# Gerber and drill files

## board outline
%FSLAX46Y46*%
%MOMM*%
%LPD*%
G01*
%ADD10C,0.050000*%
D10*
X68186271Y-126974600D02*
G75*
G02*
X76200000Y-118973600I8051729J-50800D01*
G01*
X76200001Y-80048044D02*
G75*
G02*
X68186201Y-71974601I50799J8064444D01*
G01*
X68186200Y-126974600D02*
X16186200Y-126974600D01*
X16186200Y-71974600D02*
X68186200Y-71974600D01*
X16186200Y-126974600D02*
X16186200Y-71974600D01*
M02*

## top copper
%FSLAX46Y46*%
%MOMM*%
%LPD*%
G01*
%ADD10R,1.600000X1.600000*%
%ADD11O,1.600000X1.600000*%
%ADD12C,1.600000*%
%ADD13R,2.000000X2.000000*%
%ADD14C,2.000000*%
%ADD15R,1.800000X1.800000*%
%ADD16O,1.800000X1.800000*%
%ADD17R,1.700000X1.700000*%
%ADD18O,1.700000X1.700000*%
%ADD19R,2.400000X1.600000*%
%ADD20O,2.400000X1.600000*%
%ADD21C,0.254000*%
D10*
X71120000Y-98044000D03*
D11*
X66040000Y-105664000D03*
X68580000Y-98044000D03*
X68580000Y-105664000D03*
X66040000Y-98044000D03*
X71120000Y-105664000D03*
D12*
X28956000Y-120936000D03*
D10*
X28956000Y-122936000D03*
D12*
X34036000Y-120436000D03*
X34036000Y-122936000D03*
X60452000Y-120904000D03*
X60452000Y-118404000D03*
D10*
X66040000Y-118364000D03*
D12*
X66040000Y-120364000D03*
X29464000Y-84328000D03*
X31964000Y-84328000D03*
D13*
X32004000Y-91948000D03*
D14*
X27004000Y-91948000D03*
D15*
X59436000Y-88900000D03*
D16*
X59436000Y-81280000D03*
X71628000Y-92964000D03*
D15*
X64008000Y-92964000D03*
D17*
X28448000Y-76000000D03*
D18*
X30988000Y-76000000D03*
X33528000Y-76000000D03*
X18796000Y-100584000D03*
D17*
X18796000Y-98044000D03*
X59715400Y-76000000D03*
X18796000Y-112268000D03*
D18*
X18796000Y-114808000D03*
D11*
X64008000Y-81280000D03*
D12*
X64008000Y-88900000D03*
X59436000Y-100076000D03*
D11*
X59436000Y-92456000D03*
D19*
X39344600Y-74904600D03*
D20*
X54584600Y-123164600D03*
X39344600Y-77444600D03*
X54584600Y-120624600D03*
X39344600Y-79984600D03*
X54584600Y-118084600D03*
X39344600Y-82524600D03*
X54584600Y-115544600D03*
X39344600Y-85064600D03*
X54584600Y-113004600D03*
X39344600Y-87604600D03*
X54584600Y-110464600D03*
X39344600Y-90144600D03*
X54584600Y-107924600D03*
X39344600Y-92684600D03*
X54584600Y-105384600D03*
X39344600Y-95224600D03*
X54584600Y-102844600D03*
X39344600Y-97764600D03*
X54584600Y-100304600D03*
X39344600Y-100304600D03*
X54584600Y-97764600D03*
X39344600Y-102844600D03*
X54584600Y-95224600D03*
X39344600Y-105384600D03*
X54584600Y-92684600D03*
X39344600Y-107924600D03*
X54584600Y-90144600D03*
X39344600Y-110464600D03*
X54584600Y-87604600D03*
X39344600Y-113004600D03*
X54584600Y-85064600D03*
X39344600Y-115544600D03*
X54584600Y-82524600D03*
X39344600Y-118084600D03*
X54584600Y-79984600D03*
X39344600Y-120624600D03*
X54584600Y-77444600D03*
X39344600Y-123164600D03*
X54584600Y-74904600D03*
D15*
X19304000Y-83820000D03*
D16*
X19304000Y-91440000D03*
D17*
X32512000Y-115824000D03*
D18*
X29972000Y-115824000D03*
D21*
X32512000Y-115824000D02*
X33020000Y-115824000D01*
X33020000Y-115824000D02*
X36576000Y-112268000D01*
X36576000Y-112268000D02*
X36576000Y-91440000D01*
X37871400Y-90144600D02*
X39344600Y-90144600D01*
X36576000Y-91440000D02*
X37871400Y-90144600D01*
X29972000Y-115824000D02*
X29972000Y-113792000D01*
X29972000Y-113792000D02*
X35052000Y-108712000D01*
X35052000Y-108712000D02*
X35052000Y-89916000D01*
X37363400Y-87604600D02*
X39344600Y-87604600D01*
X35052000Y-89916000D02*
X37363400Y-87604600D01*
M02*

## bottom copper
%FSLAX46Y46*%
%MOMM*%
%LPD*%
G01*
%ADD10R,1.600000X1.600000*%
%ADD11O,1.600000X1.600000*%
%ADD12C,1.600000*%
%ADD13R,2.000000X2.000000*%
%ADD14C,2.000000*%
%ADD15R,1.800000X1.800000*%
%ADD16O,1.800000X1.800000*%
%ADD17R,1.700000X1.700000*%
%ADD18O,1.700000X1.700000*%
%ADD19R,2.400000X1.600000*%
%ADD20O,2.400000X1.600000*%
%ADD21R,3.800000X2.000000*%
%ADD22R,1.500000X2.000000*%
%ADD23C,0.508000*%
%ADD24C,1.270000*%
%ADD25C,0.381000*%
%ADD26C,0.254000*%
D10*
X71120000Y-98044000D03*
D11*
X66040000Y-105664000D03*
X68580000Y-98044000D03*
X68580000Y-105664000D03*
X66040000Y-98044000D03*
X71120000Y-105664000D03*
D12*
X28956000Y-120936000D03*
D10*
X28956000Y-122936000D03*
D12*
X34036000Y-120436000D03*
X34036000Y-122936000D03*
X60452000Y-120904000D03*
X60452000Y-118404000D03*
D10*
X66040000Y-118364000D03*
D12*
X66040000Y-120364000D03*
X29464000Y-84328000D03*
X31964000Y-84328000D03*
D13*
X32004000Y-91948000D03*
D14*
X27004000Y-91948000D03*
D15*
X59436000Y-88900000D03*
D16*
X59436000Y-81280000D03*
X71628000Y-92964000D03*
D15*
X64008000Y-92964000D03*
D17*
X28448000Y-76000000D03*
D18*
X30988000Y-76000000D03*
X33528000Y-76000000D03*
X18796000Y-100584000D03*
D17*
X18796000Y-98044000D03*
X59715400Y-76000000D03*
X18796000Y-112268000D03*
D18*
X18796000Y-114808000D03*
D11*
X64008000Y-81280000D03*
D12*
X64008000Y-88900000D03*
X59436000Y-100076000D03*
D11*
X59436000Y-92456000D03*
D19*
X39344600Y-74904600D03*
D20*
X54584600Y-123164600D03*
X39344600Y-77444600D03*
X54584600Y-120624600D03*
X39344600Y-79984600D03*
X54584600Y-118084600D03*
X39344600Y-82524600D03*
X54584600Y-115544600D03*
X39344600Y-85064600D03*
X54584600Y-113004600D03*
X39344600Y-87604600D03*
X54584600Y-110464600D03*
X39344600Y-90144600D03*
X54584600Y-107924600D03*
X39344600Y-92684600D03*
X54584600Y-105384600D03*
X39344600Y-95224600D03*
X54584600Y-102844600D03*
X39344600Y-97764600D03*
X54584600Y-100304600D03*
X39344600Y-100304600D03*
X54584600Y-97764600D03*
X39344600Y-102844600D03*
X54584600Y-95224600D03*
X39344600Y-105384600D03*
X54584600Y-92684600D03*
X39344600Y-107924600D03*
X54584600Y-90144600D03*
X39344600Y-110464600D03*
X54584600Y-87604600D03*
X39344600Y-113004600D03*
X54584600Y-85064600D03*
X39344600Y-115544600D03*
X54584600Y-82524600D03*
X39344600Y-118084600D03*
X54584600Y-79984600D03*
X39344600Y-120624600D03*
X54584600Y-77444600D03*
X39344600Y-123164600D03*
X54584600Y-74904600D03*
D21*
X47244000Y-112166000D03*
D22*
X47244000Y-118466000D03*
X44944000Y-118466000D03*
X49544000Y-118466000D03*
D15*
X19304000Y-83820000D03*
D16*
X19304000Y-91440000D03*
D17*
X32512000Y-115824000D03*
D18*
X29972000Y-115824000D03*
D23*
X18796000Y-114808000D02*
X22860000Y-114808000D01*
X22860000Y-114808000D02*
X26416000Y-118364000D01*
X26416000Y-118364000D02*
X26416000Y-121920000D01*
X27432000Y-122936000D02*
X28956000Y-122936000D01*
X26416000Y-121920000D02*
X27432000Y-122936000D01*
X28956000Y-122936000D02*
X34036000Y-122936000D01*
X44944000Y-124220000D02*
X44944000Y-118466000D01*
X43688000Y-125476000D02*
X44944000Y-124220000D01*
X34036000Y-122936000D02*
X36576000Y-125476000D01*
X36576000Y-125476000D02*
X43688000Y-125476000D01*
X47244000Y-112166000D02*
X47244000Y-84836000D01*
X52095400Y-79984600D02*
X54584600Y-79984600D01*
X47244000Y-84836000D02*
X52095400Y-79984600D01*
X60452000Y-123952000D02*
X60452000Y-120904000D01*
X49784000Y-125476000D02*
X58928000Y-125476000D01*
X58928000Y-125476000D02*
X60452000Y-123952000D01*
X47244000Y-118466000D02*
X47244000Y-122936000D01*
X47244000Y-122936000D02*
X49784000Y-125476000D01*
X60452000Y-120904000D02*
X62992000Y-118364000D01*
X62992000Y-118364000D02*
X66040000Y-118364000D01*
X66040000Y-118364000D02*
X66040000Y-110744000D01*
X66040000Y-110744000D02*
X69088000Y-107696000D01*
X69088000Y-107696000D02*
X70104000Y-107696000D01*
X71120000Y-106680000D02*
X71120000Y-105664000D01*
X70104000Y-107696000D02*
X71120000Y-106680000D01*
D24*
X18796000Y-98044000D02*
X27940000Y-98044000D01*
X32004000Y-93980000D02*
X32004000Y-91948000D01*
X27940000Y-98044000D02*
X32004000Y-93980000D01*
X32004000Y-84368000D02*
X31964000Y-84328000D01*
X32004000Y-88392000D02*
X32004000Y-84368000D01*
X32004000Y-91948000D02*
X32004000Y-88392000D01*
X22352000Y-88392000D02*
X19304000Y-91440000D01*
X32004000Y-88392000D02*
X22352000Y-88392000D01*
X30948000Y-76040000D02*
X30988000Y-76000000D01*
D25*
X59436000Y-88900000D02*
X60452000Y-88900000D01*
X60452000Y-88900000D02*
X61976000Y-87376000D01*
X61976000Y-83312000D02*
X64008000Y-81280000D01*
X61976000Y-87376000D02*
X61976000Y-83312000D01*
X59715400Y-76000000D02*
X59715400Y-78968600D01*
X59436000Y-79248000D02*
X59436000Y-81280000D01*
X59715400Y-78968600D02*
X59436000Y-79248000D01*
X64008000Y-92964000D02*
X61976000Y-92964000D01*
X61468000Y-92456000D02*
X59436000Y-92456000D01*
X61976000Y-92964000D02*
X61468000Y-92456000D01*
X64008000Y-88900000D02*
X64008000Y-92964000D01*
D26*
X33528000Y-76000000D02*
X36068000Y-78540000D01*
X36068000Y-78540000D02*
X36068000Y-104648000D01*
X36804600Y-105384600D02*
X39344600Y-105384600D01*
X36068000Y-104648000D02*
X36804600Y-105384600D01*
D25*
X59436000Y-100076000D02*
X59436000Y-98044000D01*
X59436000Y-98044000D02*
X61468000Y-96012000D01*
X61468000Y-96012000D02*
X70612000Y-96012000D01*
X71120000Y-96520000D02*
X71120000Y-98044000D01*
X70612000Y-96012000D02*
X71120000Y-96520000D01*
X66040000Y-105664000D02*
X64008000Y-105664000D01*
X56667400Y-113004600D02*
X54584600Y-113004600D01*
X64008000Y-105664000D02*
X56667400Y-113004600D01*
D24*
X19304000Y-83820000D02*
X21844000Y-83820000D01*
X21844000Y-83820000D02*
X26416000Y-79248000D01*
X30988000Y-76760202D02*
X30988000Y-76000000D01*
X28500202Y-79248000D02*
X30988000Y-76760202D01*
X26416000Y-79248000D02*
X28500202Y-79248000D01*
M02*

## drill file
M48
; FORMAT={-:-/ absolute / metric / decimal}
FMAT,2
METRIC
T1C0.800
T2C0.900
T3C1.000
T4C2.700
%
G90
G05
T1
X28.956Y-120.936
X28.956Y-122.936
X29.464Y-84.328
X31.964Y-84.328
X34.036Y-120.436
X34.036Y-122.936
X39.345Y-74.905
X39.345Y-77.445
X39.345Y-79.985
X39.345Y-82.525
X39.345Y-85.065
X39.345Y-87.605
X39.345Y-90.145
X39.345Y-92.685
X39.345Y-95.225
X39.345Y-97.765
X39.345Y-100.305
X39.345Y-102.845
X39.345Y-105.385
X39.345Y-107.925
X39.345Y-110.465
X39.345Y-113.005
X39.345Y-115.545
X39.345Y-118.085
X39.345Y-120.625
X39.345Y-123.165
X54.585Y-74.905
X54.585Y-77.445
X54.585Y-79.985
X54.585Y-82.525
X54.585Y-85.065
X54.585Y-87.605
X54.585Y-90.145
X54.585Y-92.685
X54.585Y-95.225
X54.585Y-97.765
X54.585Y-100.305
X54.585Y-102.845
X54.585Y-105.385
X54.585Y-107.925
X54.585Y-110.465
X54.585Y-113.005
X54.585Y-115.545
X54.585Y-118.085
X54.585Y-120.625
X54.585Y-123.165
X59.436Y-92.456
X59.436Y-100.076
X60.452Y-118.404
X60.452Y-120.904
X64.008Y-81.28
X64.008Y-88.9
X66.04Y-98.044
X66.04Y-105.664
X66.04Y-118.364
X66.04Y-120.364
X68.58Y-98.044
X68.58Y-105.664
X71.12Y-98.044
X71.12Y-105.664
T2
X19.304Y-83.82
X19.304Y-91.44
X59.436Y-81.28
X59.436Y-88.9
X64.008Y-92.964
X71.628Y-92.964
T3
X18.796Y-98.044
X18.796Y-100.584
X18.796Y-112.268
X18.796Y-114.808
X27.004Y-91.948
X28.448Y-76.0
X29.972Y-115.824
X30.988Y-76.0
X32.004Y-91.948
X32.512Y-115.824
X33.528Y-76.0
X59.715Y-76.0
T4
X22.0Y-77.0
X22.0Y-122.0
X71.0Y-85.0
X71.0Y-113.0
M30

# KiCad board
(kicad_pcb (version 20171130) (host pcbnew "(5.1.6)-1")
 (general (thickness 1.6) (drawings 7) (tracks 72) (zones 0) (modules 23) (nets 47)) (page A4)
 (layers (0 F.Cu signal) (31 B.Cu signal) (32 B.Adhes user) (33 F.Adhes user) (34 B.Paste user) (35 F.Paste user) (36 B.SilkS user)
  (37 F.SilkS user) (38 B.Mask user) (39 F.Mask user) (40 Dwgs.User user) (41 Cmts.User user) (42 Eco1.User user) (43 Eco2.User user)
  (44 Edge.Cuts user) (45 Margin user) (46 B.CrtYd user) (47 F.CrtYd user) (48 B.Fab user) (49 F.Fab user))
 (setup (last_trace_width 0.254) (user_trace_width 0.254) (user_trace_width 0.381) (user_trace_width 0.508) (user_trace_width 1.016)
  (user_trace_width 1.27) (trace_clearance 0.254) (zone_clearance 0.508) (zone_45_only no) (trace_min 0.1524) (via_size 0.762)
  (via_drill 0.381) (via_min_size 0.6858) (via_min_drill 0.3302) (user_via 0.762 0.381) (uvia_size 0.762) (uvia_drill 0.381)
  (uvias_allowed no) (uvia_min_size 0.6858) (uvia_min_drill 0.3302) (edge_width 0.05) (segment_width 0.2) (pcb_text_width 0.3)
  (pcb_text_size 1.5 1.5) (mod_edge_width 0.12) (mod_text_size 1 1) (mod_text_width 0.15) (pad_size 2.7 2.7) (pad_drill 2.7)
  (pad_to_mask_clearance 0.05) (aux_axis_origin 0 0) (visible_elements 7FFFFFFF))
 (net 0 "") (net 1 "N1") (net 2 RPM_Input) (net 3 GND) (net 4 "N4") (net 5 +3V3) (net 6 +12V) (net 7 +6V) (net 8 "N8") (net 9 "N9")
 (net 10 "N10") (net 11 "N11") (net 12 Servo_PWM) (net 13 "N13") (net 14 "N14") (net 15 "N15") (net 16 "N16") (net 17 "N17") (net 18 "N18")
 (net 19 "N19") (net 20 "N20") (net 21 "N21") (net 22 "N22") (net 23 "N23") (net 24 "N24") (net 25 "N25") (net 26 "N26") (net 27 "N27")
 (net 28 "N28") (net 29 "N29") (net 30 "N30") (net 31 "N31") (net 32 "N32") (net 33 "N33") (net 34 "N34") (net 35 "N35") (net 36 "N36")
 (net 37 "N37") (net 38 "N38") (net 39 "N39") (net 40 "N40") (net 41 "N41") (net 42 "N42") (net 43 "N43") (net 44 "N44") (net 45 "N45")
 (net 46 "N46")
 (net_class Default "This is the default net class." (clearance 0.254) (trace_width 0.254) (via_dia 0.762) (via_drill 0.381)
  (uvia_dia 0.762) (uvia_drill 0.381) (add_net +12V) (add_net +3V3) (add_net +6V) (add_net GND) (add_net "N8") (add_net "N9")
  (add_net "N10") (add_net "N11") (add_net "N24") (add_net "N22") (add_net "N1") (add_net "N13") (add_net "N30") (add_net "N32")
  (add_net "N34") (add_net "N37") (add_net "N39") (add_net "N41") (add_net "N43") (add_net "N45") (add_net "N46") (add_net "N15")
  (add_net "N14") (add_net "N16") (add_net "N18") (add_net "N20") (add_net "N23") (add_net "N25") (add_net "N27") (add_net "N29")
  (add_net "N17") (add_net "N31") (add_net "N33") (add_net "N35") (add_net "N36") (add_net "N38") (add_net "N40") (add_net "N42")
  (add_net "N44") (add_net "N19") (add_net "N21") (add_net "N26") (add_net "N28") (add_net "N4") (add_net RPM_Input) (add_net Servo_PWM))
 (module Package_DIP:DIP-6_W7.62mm (layer F.Cu) (at 71.12 98.044 270)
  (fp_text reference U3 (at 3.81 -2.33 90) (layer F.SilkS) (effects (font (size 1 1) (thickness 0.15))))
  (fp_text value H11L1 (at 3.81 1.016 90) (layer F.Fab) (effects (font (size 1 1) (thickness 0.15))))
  (pad 1 thru_hole rect (at 0 0 270) (size 1.6 1.6) (drill 0.8) (layers *.Cu *.Mask) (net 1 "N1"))
  (pad 4 thru_hole oval (at 7.62 5.08 270) (size 1.6 1.6) (drill 0.8) (layers *.Cu *.Mask) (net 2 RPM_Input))
  (pad 2 thru_hole oval (at 0 2.54 270) (size 1.6 1.6) (drill 0.8) (layers *.Cu *.Mask) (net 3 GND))
  (pad 5 thru_hole oval (at 7.62 2.54 270) (size 1.6 1.6) (drill 0.8) (layers *.Cu *.Mask) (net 3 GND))
  (pad 3 thru_hole oval (at 0 5.08 270) (size 1.6 1.6) (drill 0.8) (layers *.Cu *.Mask) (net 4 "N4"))
  (pad 6 thru_hole oval (at 7.62 0 270) (size 1.6 1.6) (drill 0.8) (layers *.Cu *.Mask) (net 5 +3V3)))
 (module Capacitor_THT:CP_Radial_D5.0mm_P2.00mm (layer F.Cu) (at 28.956 122.936 90)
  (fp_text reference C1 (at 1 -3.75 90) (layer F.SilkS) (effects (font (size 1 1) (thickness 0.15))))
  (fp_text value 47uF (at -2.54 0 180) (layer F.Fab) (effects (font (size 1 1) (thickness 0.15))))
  (pad 2 thru_hole circle (at 2 0 90) (size 1.6 1.6) (drill 0.8) (layers *.Cu *.Mask) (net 3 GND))
  (pad 1 thru_hole rect (at 0 0 90) (size 1.6 1.6) (drill 0.8) (layers *.Cu *.Mask) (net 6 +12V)))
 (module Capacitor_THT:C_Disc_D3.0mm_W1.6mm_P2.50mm (layer F.Cu) (at 34.036 122.936 90)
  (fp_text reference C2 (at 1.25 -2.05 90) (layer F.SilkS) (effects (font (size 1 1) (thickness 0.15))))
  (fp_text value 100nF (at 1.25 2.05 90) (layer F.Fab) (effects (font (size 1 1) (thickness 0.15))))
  (pad 2 thru_hole circle (at 2.5 0 90) (size 1.6 1.6) (drill 0.8) (layers *.Cu *.Mask) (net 3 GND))
  (pad 1 thru_hole circle (at 0 0 90) (size 1.6 1.6) (drill 0.8) (layers *.Cu *.Mask) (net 6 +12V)))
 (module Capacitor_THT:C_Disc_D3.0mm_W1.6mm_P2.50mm (layer F.Cu) (at 60.452 120.904 90)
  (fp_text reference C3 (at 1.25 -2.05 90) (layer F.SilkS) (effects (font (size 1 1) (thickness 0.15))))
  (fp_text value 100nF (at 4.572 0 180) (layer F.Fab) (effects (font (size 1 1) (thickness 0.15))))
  (pad 1 thru_hole circle (at 0 0 90) (size 1.6 1.6) (drill 0.8) (layers *.Cu *.Mask) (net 5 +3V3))
  (pad 2 thru_hole circle (at 2.5 0 90) (size 1.6 1.6) (drill 0.8) (layers *.Cu *.Mask) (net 3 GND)))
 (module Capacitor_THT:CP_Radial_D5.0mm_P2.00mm (layer F.Cu) (at 66.04 118.364 270)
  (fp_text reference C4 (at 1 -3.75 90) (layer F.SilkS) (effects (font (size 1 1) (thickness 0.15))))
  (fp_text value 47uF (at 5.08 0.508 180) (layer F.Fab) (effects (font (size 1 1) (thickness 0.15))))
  (pad 1 thru_hole rect (at 0 0 270) (size 1.6 1.6) (drill 0.8) (layers *.Cu *.Mask) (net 5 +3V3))
  (pad 2 thru_hole circle (at 2 0 270) (size 1.6 1.6) (drill 0.8) (layers *.Cu *.Mask) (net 3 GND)))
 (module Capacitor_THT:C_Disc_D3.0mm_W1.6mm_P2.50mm (layer F.Cu) (at 29.464 84.328)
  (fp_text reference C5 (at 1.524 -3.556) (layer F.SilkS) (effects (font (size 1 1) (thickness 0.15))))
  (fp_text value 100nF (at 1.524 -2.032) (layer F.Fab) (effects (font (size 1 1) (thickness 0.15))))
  (pad 1 thru_hole circle (at 0 0) (size 1.6 1.6) (drill 0.8) (layers *.Cu *.Mask) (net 3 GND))
  (pad 2 thru_hole circle (at 2.5 0) (size 1.6 1.6) (drill 0.8) (layers *.Cu *.Mask) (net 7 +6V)))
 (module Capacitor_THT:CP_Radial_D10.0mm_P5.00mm (layer F.Cu) (at 32.004 91.948 180)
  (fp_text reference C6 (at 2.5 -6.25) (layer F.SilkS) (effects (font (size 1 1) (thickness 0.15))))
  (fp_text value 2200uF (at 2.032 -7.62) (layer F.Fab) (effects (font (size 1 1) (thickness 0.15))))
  (pad 1 thru_hole rect (at 0 0 180) (size 2 2) (drill 1) (layers *.Cu *.Mask) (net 7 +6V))
  (pad 2 thru_hole circle (at 5 0 180) (size 2 2) (drill 1) (layers *.Cu *.Mask) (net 3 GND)))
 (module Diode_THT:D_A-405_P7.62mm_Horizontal (layer F.Cu) (at 59.436 88.9 90)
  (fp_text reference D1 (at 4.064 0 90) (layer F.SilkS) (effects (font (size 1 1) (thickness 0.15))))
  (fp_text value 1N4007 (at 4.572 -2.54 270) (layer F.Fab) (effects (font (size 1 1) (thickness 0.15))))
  (pad 1 thru_hole rect (at 0 0 90) (size 1.8 1.8) (drill 0.9) (layers *.Cu *.Mask) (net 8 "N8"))
  (pad 2 thru_hole oval (at 7.62 0 90) (size 1.8 1.8) (drill 0.9) (layers *.Cu *.Mask) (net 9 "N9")))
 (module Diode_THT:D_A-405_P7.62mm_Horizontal (layer F.Cu) (at 64.008 92.964)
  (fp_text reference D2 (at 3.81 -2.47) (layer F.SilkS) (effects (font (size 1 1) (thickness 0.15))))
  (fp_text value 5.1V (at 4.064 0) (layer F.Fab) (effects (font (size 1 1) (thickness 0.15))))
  (pad 2 thru_hole oval (at 7.62 0) (size 1.8 1.8) (drill 0.9) (layers *.Cu *.Mask) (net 3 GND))
  (pad 1 thru_hole rect (at 0 0) (size 1.8 1.8) (drill 0.9) (layers *.Cu *.Mask) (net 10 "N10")))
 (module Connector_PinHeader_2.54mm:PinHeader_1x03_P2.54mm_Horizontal (layer F.Cu) (at 28.448 76 90)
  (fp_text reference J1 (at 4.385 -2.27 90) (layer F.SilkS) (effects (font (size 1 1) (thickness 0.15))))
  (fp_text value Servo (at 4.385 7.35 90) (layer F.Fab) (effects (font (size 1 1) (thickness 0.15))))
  (pad 1 thru_hole rect (at 0 0 90) (size 1.7 1.7) (drill 1) (layers *.Cu *.Mask) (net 3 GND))
  (pad 2 thru_hole oval (at 0 2.54 90) (size 1.7 1.7) (drill 1) (layers *.Cu *.Mask) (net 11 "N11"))
  (pad 3 thru_hole oval (at 0 5.08 90) (size 1.7 1.7) (drill 1) (layers *.Cu *.Mask) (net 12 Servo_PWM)))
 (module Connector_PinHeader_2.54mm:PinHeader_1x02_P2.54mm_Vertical (layer F.Cu) (at 18.796 98.044)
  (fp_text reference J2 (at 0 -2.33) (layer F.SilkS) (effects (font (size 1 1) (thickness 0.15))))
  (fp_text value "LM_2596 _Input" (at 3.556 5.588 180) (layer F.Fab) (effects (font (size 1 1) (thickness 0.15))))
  (pad 2 thru_hole oval (at 0 2.54) (size 1.7 1.7) (drill 1) (layers *.Cu *.Mask) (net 3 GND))
  (pad 1 thru_hole rect (at 0 0) (size 1.7 1.7) (drill 1) (layers *.Cu *.Mask) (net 7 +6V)))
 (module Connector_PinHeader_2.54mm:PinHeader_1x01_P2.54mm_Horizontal (layer F.Cu) (at 59.7154 76 90)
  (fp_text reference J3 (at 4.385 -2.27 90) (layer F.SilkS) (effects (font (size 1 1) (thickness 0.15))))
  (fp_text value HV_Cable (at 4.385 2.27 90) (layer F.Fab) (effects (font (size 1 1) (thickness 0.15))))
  (pad 1 thru_hole rect (at 0 0 90) (size 1.7 1.7) (drill 1) (layers *.Cu *.Mask) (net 9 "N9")))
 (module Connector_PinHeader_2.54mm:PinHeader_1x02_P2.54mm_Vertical (layer F.Cu) (at 18.796 112.268)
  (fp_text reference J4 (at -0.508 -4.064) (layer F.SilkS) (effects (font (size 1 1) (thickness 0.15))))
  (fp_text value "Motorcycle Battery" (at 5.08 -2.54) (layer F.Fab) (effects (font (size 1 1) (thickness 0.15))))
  (pad 1 thru_hole rect (at 0 0) (size 1.7 1.7) (drill 1) (layers *.Cu *.Mask) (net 3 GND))
  (pad 2 thru_hole oval (at 0 2.54) (size 1.7 1.7) (drill 1) (layers *.Cu *.Mask) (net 6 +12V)))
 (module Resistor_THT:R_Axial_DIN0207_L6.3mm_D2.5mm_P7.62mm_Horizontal (layer F.Cu) (at 64.008 88.9 90)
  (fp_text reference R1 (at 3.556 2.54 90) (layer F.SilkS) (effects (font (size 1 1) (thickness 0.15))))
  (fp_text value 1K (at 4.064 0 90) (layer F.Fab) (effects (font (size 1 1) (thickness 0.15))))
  (pad 2 thru_hole oval (at 7.62 0 90) (size 1.6 1.6) (drill 0.8) (layers *.Cu *.Mask) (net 8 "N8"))
  (pad 1 thru_hole circle (at 0 0 90) (size 1.6 1.6) (drill 0.8) (layers *.Cu *.Mask) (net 10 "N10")))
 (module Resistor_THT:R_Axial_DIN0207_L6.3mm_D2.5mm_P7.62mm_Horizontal (layer F.Cu) (at 59.436 100.076 90)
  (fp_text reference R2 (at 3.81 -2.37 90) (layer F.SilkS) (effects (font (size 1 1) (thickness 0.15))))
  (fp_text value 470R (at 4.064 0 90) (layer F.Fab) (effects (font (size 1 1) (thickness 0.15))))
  (pad 1 thru_hole circle (at 0 0 90) (size 1.6 1.6) (drill 0.8) (layers *.Cu *.Mask) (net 1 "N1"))
  (pad 2 thru_hole oval (at 7.62 0 90) (size 1.6 1.6) (drill 0.8) (layers *.Cu *.Mask) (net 10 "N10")))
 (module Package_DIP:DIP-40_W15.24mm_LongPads (layer F.Cu) (at 39.3446 74.9046)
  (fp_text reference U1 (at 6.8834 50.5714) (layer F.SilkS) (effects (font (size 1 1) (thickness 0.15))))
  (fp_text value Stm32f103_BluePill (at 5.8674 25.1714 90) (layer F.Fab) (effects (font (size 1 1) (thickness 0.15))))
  (pad 1 thru_hole rect (at 0 0) (size 2.4 1.6) (drill 0.8) (layers *.Cu *.Mask) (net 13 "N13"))
  (pad 21 thru_hole oval (at 15.24 48.26) (size 2.4 1.6) (drill 0.8) (layers *.Cu *.Mask) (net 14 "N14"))
  (pad 2 thru_hole oval (at 0 2.54) (size 2.4 1.6) (drill 0.8) (layers *.Cu *.Mask) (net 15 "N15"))
  (pad 22 thru_hole oval (at 15.24 45.72) (size 2.4 1.6) (drill 0.8) (layers *.Cu *.Mask) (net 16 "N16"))
  (pad 3 thru_hole oval (at 0 5.08) (size 2.4 1.6) (drill 0.8) (layers *.Cu *.Mask) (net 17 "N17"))
  (pad 23 thru_hole oval (at 15.24 43.18) (size 2.4 1.6) (drill 0.8) (layers *.Cu *.Mask) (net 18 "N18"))
  (pad 4 thru_hole oval (at 0 7.62) (size 2.4 1.6) (drill 0.8) (layers *.Cu *.Mask) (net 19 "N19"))
  (pad 24 thru_hole oval (at 15.24 40.64) (size 2.4 1.6) (drill 0.8) (layers *.Cu *.Mask) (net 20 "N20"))
  (pad 5 thru_hole oval (at 0 10.16) (size 2.4 1.6) (drill 0.8) (layers *.Cu *.Mask) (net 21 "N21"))
  (pad 25 thru_hole oval (at 15.24 38.1) (size 2.4 1.6) (drill 0.8) (layers *.Cu *.Mask) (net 2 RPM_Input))
  (pad 6 thru_hole oval (at 0 12.7) (size 2.4 1.6) (drill 0.8) (layers *.Cu *.Mask) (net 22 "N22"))
  (pad 26 thru_hole oval (at 15.24 35.56) (size 2.4 1.6) (drill 0.8) (layers *.Cu *.Mask) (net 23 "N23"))
  (pad 7 thru_hole oval (at 0 15.24) (size 2.4 1.6) (drill 0.8) (layers *.Cu *.Mask) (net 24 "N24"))
  (pad 27 thru_hole oval (at 15.24 33.02) (size 2.4 1.6) (drill 0.8) (layers *.Cu *.Mask) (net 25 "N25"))
  (pad 8 thru_hole oval (at 0 17.78) (size 2.4 1.6) (drill 0.8) (layers *.Cu *.Mask) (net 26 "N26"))
  (pad 28 thru_hole oval (at 15.24 30.48) (size 2.4 1.6) (drill 0.8) (layers *.Cu *.Mask) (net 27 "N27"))
  (pad 9 thru_hole oval (at 0 20.32) (size 2.4 1.6) (drill 0.8) (layers *.Cu *.Mask) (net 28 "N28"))
  (pad 29 thru_hole oval (at 15.24 27.94) (size 2.4 1.6) (drill 0.8) (layers *.Cu *.Mask) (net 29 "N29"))
  (pad 10 thru_hole oval (at 0 22.86) (size 2.4 1.6) (drill 0.8) (layers *.Cu *.Mask) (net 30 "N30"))
  (pad 30 thru_hole oval (at 15.24 25.4) (size 2.4 1.6) (drill 0.8) (layers *.Cu *.Mask) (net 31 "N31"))
  (pad 11 thru_hole oval (at 0 25.4) (size 2.4 1.6) (drill 0.8) (layers *.Cu *.Mask) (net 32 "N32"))
  (pad 31 thru_hole oval (at 15.24 22.86) (size 2.4 1.6) (drill 0.8) (layers *.Cu *.Mask) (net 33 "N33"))
  (pad 12 thru_hole oval (at 0 27.94) (size 2.4 1.6) (drill 0.8) (layers *.Cu *.Mask) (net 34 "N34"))
  (pad 32 thru_hole oval (at 15.24 20.32) (size 2.4 1.6) (drill 0.8) (layers *.Cu *.Mask) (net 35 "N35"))
  (pad 13 thru_hole oval (at 0 30.48) (size 2.4 1.6) (drill 0.8) (layers *.Cu *.Mask) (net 12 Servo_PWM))
  (pad 33 thru_hole oval (at 15.24 17.78) (size 2.4 1.6) (drill 0.8) (layers *.Cu *.Mask) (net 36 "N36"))
  (pad 14 thru_hole oval (at 0 33.02) (size 2.4 1.6) (drill 0.8) (layers *.Cu *.Mask) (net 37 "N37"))
  (pad 34 thru_hole oval (at 15.24 15.24) (size 2.4 1.6) (drill 0.8) (layers *.Cu *.Mask) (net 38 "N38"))
  (pad 15 thru_hole oval (at 0 35.56) (size 2.4 1.6) (drill 0.8) (layers *.Cu *.Mask) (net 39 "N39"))
  (pad 35 thru_hole oval (at 15.24 12.7) (size 2.4 1.6) (drill 0.8) (layers *.Cu *.Mask) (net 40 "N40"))
  (pad 16 thru_hole oval (at 0 38.1) (size 2.4 1.6) (drill 0.8) (layers *.Cu *.Mask) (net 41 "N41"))
  (pad 36 thru_hole oval (at 15.24 10.16) (size 2.4 1.6) (drill 0.8) (layers *.Cu *.Mask) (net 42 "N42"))
  (pad 17 thru_hole oval (at 0 40.64) (size 2.4 1.6) (drill 0.8) (layers *.Cu *.Mask) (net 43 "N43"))
  (pad 37 thru_hole oval (at 15.24 7.62) (size 2.4 1.6) (drill 0.8) (layers *.Cu *.Mask) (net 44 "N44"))
  (pad 18 thru_hole oval (at 0 43.18) (size 2.4 1.6) (drill 0.8) (layers *.Cu *.Mask) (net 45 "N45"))
  (pad 38 thru_hole oval (at 15.24 5.08) (size 2.4 1.6) (drill 0.8) (layers *.Cu *.Mask) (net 5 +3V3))
  (pad 19 thru_hole oval (at 0 45.72) (size 2.4 1.6) (drill 0.8) (layers *.Cu *.Mask) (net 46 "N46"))
  (pad 39 thru_hole oval (at 15.24 2.54) (size 2.4 1.6) (drill 0.8) (layers *.Cu *.Mask) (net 3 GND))
  (pad 20 thru_hole oval (at 0 48.26) (size 2.4 1.6) (drill 0.8) (layers *.Cu *.Mask) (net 5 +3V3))
  (pad 40 thru_hole oval (at 15.24 0) (size 2.4 1.6) (drill 0.8) (layers *.Cu *.Mask) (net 3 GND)))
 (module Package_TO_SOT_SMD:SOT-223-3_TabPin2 (layer B.Cu) (at 47.244 115.316 90)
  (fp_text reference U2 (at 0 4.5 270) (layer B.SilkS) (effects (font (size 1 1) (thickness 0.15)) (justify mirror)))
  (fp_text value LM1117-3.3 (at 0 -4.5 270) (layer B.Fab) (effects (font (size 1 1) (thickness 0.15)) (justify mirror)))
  (pad 2 smd rect (at 3.15 0 90) (size 2 3.8) (layers B.Cu B.Paste B.Mask) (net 5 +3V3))
  (pad 2 smd rect (at -3.15 0 90) (size 2 1.5) (layers B.Cu B.Paste B.Mask) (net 5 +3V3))
  (pad 3 smd rect (at -3.15 -2.3 90) (size 2 1.5) (layers B.Cu B.Paste B.Mask) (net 6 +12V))
  (pad 1 smd rect (at -3.15 2.3 90) (size 2 1.5) (layers B.Cu B.Paste B.Mask) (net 3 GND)))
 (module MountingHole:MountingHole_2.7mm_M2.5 (layer F.Cu) (at 71 85)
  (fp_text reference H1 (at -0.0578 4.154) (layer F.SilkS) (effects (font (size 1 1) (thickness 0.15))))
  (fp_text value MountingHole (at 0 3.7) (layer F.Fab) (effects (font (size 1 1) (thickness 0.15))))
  (pad 1 np_thru_hole circle (at 0 0) (size 2.7 2.7) (drill 2.7) (layers *.Cu *.Mask)))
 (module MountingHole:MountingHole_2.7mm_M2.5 (layer F.Cu) (at 71 113)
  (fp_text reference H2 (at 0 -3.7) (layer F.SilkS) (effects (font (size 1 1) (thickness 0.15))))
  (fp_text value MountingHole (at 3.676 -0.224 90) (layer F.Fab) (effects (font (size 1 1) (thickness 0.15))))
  (pad 1 np_thru_hole circle (at 0 0) (size 2.7 2.7) (drill 2.7) (layers *.Cu *.Mask)))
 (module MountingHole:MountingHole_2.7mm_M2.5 (layer F.Cu) (at 22 77)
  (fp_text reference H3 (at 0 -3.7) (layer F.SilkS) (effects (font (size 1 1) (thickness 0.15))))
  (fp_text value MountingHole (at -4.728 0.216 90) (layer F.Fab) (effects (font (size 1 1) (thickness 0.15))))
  (pad 1 np_thru_hole circle (at 0 0) (size 2.7 2.7) (drill 2.7) (layers *.Cu *.Mask)))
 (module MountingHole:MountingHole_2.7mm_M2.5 (layer F.Cu) (at 22 122)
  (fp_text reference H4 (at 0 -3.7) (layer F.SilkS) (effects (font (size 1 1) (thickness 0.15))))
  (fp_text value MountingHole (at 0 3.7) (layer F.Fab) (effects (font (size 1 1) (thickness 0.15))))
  (pad 1 np_thru_hole circle (at 0 0) (size 2.7 2.7) (drill 2.7) (layers *.Cu *.Mask)))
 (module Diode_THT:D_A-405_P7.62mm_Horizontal (layer F.Cu) (at 19.304 83.82 270)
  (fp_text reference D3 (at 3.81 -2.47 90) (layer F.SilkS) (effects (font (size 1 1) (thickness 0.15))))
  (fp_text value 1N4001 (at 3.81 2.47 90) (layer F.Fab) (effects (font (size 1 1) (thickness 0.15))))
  (pad 1 thru_hole rect (at 0 0 270) (size 1.8 1.8) (drill 0.9) (layers *.Cu *.Mask) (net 11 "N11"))
  (pad 2 thru_hole oval (at 7.62 0 270) (size 1.8 1.8) (drill 0.9) (layers *.Cu *.Mask) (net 7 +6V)))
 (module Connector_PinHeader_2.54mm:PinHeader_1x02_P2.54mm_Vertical (layer F.Cu) (at 32.512 115.824 270)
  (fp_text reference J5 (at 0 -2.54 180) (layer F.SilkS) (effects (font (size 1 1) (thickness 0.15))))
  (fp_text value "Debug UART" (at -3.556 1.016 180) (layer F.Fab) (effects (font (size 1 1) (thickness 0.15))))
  (pad 1 thru_hole rect (at 0 0 270) (size 1.7 1.7) (drill 1) (layers *.Cu *.Mask) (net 24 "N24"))
  (pad 2 thru_hole oval (at 0 2.54 270) (size 1.7 1.7) (drill 1) (layers *.Cu *.Mask) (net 22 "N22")))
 (gr_arc (start 76.238 127.0254) (end 76.2 118.9736) (angle -89.36811196) (layer Edge.Cuts) (width 0.05))
 (gr_arc (start 76.2508 71.9836) (end 68.186201 71.974601) (angle -89.70302521) (layer Edge.Cuts) (width 0.05))
 (gr_line (start 68.1862 126.9746) (end 16.1862 126.9746) (layer Edge.Cuts) (width 0.05))
 (gr_line (start 16.1862 71.9746) (end 68.1862 71.9746) (layer Edge.Cuts) (width 0.05))
 (gr_line (start 16.1862 126.9746) (end 16.1862 71.9746) (layer Edge.Cuts) (width 0.05))
 (segment (start 18.796 114.808) (end 22.86 114.808) (width 0.508) (layer B.Cu) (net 6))
 (segment (start 22.86 114.808) (end 26.416 118.364) (width 0.508) (layer B.Cu) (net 6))
 (segment (start 26.416 118.364) (end 26.416 121.92) (width 0.508) (layer B.Cu) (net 6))
 (segment (start 27.432 122.936) (end 28.956 122.936) (width 0.508) (layer B.Cu) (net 6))
 (segment (start 26.416 121.92) (end 27.432 122.936) (width 0.508) (layer B.Cu) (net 6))
 (segment (start 28.956 122.936) (end 34.036 122.936) (width 0.508) (layer B.Cu) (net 6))
 (segment (start 44.944 124.22) (end 44.944 118.466) (width 0.508) (layer B.Cu) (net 6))
 (segment (start 43.688 125.476) (end 44.944 124.22) (width 0.508) (layer B.Cu) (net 6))
 (segment (start 34.036 122.936) (end 36.576 125.476) (width 0.508) (layer B.Cu) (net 6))
 (segment (start 36.576 125.476) (end 43.688 125.476) (width 0.508) (layer B.Cu) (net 6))
 (segment (start 47.244 112.166) (end 47.244 84.836) (width 0.508) (layer B.Cu) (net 5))
 (segment (start 52.0954 79.9846) (end 54.5846 79.9846) (width 0.508) (layer B.Cu) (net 5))
 (segment (start 47.244 84.836) (end 52.0954 79.9846) (width 0.508) (layer B.Cu) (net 5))
 (segment (start 60.452 123.952) (end 60.452 120.904) (width 0.508) (layer B.Cu) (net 5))
 (segment (start 49.784 125.476) (end 58.928 125.476) (width 0.508) (layer B.Cu) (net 5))
 (segment (start 58.928 125.476) (end 60.452 123.952) (width 0.508) (layer B.Cu) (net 5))
 (segment (start 47.244 118.466) (end 47.244 122.936) (width 0.508) (layer B.Cu) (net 5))
 (segment (start 47.244 122.936) (end 49.784 125.476) (width 0.508) (layer B.Cu) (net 5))
 (segment (start 60.452 120.904) (end 62.992 118.364) (width 0.508) (layer B.Cu) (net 5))
 (segment (start 62.992 118.364) (end 66.04 118.364) (width 0.508) (layer B.Cu) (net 5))
 (segment (start 66.04 118.364) (end 66.04 110.744) (width 0.508) (layer B.Cu) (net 5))
 (segment (start 66.04 110.744) (end 69.088 107.696) (width 0.508) (layer B.Cu) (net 5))
 (segment (start 69.088 107.696) (end 70.104 107.696) (width 0.508) (layer B.Cu) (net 5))
 (segment (start 71.12 106.68) (end 71.12 105.664) (width 0.508) (layer B.Cu) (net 5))
 (segment (start 70.104 107.696) (end 71.12 106.68) (width 0.508) (layer B.Cu) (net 5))
 (segment (start 18.796 98.044) (end 27.94 98.044) (width 1.27) (layer B.Cu) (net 7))
 (segment (start 32.004 93.98) (end 32.004 91.948) (width 1.27) (layer B.Cu) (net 7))
 (segment (start 27.94 98.044) (end 32.004 93.98) (width 1.27) (layer B.Cu) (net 7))
 (segment (start 32.004 84.368) (end 31.964 84.328) (width 1.27) (layer B.Cu) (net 7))
 (segment (start 32.004 88.392) (end 32.004 84.368) (width 1.27) (layer B.Cu) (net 7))
 (segment (start 32.004 91.948) (end 32.004 88.392) (width 1.27) (layer B.Cu) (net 7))
 (segment (start 22.352 88.392) (end 19.304 91.44) (width 1.27) (layer B.Cu) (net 7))
 (segment (start 32.004 88.392) (end 22.352 88.392) (width 1.27) (layer B.Cu) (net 7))
 (segment (start 30.948 76.04) (end 30.988 76) (width 1.27) (layer B.Cu) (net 11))
 (segment (start 59.436 88.9) (end 60.452 88.9) (width 0.381) (layer B.Cu) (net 8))
 (segment (start 60.452 88.9) (end 61.976 87.376) (width 0.381) (layer B.Cu) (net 8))
 (segment (start 61.976 83.312) (end 64.008 81.28) (width 0.381) (layer B.Cu) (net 8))
 (segment (start 61.976 87.376) (end 61.976 83.312) (width 0.381) (layer B.Cu) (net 8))
 (segment (start 59.7154 76) (end 59.7154 78.9686) (width 0.381) (layer B.Cu) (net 9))
 (segment (start 59.436 79.248) (end 59.436 81.28) (width 0.381) (layer B.Cu) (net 9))
 (segment (start 59.7154 78.9686) (end 59.436 79.248) (width 0.381) (layer B.Cu) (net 9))
 (segment (start 64.008 92.964) (end 61.976 92.964) (width 0.381) (layer B.Cu) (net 10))
 (segment (start 61.468 92.456) (end 59.436 92.456) (width 0.381) (layer B.Cu) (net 10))
 (segment (start 61.976 92.964) (end 61.468 92.456) (width 0.381) (layer B.Cu) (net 10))
 (segment (start 64.008 88.9) (end 64.008 92.964) (width 0.381) (layer B.Cu) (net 10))
 (segment (start 33.528 76) (end 36.068 78.54) (width 0.254) (layer B.Cu) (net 12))
 (segment (start 36.068 78.54) (end 36.068 104.648) (width 0.254) (layer B.Cu) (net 12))
 (segment (start 36.8046 105.3846) (end 39.3446 105.3846) (width 0.254) (layer B.Cu) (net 12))
 (segment (start 36.068 104.648) (end 36.8046 105.3846) (width 0.254) (layer B.Cu) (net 12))
 (segment (start 59.436 100.076) (end 59.436 98.044) (width 0.381) (layer B.Cu) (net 1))
 (segment (start 59.436 98.044) (end 61.468 96.012) (width 0.381) (layer B.Cu) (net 1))
 (segment (start 61.468 96.012) (end 70.612 96.012) (width 0.381) (layer B.Cu) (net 1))
 (segment (start 71.12 96.52) (end 71.12 98.044) (width 0.381) (layer B.Cu) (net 1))
 (segment (start 70.612 96.012) (end 71.12 96.52) (width 0.381) (layer B.Cu) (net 1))
 (segment (start 66.04 105.664) (end 64.008 105.664) (width 0.381) (layer B.Cu) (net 2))
 (segment (start 56.6674 113.0046) (end 54.5846 113.0046) (width 0.381) (layer B.Cu) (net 2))
 (segment (start 64.008 105.664) (end 56.6674 113.0046) (width 0.381) (layer B.Cu) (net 2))
 (segment (start 19.304 83.82) (end 21.844 83.82) (width 1.27) (layer B.Cu) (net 11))
 (segment (start 21.844 83.82) (end 26.416 79.248) (width 1.27) (layer B.Cu) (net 11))
 (segment (start 30.988 76.760202) (end 30.988 76) (width 1.27) (layer B.Cu) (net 11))
 (segment (start 28.500202 79.248) (end 30.988 76.760202) (width 1.27) (layer B.Cu) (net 11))
 (segment (start 26.416 79.248) (end 28.500202 79.248) (width 1.27) (layer B.Cu) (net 11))
 (segment (start 32.512 115.824) (end 33.02 115.824) (width 0.254) (layer F.Cu) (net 24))
 (segment (start 33.02 115.824) (end 36.576 112.268) (width 0.254) (layer F.Cu) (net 24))
 (segment (start 36.576 112.268) (end 36.576 91.44) (width 0.254) (layer F.Cu) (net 24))
 (segment (start 37.8714 90.1446) (end 39.3446 90.1446) (width 0.254) (layer F.Cu) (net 24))
 (segment (start 36.576 91.44) (end 37.8714 90.1446) (width 0.254) (layer F.Cu) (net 24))
 (segment (start 29.972 115.824) (end 29.972 113.792) (width 0.254) (layer F.Cu) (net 22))
 (segment (start 29.972 113.792) (end 35.052 108.712) (width 0.254) (layer F.Cu) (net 22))
 (segment (start 35.052 108.712) (end 35.052 89.916) (width 0.254) (layer F.Cu) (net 22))
 (segment (start 37.3634 87.6046) (end 39.3446 87.6046) (width 0.254) (layer F.Cu) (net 22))
 (segment (start 35.052 89.916) (end 37.3634 87.6046) (width 0.254) (layer F.Cu) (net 22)))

